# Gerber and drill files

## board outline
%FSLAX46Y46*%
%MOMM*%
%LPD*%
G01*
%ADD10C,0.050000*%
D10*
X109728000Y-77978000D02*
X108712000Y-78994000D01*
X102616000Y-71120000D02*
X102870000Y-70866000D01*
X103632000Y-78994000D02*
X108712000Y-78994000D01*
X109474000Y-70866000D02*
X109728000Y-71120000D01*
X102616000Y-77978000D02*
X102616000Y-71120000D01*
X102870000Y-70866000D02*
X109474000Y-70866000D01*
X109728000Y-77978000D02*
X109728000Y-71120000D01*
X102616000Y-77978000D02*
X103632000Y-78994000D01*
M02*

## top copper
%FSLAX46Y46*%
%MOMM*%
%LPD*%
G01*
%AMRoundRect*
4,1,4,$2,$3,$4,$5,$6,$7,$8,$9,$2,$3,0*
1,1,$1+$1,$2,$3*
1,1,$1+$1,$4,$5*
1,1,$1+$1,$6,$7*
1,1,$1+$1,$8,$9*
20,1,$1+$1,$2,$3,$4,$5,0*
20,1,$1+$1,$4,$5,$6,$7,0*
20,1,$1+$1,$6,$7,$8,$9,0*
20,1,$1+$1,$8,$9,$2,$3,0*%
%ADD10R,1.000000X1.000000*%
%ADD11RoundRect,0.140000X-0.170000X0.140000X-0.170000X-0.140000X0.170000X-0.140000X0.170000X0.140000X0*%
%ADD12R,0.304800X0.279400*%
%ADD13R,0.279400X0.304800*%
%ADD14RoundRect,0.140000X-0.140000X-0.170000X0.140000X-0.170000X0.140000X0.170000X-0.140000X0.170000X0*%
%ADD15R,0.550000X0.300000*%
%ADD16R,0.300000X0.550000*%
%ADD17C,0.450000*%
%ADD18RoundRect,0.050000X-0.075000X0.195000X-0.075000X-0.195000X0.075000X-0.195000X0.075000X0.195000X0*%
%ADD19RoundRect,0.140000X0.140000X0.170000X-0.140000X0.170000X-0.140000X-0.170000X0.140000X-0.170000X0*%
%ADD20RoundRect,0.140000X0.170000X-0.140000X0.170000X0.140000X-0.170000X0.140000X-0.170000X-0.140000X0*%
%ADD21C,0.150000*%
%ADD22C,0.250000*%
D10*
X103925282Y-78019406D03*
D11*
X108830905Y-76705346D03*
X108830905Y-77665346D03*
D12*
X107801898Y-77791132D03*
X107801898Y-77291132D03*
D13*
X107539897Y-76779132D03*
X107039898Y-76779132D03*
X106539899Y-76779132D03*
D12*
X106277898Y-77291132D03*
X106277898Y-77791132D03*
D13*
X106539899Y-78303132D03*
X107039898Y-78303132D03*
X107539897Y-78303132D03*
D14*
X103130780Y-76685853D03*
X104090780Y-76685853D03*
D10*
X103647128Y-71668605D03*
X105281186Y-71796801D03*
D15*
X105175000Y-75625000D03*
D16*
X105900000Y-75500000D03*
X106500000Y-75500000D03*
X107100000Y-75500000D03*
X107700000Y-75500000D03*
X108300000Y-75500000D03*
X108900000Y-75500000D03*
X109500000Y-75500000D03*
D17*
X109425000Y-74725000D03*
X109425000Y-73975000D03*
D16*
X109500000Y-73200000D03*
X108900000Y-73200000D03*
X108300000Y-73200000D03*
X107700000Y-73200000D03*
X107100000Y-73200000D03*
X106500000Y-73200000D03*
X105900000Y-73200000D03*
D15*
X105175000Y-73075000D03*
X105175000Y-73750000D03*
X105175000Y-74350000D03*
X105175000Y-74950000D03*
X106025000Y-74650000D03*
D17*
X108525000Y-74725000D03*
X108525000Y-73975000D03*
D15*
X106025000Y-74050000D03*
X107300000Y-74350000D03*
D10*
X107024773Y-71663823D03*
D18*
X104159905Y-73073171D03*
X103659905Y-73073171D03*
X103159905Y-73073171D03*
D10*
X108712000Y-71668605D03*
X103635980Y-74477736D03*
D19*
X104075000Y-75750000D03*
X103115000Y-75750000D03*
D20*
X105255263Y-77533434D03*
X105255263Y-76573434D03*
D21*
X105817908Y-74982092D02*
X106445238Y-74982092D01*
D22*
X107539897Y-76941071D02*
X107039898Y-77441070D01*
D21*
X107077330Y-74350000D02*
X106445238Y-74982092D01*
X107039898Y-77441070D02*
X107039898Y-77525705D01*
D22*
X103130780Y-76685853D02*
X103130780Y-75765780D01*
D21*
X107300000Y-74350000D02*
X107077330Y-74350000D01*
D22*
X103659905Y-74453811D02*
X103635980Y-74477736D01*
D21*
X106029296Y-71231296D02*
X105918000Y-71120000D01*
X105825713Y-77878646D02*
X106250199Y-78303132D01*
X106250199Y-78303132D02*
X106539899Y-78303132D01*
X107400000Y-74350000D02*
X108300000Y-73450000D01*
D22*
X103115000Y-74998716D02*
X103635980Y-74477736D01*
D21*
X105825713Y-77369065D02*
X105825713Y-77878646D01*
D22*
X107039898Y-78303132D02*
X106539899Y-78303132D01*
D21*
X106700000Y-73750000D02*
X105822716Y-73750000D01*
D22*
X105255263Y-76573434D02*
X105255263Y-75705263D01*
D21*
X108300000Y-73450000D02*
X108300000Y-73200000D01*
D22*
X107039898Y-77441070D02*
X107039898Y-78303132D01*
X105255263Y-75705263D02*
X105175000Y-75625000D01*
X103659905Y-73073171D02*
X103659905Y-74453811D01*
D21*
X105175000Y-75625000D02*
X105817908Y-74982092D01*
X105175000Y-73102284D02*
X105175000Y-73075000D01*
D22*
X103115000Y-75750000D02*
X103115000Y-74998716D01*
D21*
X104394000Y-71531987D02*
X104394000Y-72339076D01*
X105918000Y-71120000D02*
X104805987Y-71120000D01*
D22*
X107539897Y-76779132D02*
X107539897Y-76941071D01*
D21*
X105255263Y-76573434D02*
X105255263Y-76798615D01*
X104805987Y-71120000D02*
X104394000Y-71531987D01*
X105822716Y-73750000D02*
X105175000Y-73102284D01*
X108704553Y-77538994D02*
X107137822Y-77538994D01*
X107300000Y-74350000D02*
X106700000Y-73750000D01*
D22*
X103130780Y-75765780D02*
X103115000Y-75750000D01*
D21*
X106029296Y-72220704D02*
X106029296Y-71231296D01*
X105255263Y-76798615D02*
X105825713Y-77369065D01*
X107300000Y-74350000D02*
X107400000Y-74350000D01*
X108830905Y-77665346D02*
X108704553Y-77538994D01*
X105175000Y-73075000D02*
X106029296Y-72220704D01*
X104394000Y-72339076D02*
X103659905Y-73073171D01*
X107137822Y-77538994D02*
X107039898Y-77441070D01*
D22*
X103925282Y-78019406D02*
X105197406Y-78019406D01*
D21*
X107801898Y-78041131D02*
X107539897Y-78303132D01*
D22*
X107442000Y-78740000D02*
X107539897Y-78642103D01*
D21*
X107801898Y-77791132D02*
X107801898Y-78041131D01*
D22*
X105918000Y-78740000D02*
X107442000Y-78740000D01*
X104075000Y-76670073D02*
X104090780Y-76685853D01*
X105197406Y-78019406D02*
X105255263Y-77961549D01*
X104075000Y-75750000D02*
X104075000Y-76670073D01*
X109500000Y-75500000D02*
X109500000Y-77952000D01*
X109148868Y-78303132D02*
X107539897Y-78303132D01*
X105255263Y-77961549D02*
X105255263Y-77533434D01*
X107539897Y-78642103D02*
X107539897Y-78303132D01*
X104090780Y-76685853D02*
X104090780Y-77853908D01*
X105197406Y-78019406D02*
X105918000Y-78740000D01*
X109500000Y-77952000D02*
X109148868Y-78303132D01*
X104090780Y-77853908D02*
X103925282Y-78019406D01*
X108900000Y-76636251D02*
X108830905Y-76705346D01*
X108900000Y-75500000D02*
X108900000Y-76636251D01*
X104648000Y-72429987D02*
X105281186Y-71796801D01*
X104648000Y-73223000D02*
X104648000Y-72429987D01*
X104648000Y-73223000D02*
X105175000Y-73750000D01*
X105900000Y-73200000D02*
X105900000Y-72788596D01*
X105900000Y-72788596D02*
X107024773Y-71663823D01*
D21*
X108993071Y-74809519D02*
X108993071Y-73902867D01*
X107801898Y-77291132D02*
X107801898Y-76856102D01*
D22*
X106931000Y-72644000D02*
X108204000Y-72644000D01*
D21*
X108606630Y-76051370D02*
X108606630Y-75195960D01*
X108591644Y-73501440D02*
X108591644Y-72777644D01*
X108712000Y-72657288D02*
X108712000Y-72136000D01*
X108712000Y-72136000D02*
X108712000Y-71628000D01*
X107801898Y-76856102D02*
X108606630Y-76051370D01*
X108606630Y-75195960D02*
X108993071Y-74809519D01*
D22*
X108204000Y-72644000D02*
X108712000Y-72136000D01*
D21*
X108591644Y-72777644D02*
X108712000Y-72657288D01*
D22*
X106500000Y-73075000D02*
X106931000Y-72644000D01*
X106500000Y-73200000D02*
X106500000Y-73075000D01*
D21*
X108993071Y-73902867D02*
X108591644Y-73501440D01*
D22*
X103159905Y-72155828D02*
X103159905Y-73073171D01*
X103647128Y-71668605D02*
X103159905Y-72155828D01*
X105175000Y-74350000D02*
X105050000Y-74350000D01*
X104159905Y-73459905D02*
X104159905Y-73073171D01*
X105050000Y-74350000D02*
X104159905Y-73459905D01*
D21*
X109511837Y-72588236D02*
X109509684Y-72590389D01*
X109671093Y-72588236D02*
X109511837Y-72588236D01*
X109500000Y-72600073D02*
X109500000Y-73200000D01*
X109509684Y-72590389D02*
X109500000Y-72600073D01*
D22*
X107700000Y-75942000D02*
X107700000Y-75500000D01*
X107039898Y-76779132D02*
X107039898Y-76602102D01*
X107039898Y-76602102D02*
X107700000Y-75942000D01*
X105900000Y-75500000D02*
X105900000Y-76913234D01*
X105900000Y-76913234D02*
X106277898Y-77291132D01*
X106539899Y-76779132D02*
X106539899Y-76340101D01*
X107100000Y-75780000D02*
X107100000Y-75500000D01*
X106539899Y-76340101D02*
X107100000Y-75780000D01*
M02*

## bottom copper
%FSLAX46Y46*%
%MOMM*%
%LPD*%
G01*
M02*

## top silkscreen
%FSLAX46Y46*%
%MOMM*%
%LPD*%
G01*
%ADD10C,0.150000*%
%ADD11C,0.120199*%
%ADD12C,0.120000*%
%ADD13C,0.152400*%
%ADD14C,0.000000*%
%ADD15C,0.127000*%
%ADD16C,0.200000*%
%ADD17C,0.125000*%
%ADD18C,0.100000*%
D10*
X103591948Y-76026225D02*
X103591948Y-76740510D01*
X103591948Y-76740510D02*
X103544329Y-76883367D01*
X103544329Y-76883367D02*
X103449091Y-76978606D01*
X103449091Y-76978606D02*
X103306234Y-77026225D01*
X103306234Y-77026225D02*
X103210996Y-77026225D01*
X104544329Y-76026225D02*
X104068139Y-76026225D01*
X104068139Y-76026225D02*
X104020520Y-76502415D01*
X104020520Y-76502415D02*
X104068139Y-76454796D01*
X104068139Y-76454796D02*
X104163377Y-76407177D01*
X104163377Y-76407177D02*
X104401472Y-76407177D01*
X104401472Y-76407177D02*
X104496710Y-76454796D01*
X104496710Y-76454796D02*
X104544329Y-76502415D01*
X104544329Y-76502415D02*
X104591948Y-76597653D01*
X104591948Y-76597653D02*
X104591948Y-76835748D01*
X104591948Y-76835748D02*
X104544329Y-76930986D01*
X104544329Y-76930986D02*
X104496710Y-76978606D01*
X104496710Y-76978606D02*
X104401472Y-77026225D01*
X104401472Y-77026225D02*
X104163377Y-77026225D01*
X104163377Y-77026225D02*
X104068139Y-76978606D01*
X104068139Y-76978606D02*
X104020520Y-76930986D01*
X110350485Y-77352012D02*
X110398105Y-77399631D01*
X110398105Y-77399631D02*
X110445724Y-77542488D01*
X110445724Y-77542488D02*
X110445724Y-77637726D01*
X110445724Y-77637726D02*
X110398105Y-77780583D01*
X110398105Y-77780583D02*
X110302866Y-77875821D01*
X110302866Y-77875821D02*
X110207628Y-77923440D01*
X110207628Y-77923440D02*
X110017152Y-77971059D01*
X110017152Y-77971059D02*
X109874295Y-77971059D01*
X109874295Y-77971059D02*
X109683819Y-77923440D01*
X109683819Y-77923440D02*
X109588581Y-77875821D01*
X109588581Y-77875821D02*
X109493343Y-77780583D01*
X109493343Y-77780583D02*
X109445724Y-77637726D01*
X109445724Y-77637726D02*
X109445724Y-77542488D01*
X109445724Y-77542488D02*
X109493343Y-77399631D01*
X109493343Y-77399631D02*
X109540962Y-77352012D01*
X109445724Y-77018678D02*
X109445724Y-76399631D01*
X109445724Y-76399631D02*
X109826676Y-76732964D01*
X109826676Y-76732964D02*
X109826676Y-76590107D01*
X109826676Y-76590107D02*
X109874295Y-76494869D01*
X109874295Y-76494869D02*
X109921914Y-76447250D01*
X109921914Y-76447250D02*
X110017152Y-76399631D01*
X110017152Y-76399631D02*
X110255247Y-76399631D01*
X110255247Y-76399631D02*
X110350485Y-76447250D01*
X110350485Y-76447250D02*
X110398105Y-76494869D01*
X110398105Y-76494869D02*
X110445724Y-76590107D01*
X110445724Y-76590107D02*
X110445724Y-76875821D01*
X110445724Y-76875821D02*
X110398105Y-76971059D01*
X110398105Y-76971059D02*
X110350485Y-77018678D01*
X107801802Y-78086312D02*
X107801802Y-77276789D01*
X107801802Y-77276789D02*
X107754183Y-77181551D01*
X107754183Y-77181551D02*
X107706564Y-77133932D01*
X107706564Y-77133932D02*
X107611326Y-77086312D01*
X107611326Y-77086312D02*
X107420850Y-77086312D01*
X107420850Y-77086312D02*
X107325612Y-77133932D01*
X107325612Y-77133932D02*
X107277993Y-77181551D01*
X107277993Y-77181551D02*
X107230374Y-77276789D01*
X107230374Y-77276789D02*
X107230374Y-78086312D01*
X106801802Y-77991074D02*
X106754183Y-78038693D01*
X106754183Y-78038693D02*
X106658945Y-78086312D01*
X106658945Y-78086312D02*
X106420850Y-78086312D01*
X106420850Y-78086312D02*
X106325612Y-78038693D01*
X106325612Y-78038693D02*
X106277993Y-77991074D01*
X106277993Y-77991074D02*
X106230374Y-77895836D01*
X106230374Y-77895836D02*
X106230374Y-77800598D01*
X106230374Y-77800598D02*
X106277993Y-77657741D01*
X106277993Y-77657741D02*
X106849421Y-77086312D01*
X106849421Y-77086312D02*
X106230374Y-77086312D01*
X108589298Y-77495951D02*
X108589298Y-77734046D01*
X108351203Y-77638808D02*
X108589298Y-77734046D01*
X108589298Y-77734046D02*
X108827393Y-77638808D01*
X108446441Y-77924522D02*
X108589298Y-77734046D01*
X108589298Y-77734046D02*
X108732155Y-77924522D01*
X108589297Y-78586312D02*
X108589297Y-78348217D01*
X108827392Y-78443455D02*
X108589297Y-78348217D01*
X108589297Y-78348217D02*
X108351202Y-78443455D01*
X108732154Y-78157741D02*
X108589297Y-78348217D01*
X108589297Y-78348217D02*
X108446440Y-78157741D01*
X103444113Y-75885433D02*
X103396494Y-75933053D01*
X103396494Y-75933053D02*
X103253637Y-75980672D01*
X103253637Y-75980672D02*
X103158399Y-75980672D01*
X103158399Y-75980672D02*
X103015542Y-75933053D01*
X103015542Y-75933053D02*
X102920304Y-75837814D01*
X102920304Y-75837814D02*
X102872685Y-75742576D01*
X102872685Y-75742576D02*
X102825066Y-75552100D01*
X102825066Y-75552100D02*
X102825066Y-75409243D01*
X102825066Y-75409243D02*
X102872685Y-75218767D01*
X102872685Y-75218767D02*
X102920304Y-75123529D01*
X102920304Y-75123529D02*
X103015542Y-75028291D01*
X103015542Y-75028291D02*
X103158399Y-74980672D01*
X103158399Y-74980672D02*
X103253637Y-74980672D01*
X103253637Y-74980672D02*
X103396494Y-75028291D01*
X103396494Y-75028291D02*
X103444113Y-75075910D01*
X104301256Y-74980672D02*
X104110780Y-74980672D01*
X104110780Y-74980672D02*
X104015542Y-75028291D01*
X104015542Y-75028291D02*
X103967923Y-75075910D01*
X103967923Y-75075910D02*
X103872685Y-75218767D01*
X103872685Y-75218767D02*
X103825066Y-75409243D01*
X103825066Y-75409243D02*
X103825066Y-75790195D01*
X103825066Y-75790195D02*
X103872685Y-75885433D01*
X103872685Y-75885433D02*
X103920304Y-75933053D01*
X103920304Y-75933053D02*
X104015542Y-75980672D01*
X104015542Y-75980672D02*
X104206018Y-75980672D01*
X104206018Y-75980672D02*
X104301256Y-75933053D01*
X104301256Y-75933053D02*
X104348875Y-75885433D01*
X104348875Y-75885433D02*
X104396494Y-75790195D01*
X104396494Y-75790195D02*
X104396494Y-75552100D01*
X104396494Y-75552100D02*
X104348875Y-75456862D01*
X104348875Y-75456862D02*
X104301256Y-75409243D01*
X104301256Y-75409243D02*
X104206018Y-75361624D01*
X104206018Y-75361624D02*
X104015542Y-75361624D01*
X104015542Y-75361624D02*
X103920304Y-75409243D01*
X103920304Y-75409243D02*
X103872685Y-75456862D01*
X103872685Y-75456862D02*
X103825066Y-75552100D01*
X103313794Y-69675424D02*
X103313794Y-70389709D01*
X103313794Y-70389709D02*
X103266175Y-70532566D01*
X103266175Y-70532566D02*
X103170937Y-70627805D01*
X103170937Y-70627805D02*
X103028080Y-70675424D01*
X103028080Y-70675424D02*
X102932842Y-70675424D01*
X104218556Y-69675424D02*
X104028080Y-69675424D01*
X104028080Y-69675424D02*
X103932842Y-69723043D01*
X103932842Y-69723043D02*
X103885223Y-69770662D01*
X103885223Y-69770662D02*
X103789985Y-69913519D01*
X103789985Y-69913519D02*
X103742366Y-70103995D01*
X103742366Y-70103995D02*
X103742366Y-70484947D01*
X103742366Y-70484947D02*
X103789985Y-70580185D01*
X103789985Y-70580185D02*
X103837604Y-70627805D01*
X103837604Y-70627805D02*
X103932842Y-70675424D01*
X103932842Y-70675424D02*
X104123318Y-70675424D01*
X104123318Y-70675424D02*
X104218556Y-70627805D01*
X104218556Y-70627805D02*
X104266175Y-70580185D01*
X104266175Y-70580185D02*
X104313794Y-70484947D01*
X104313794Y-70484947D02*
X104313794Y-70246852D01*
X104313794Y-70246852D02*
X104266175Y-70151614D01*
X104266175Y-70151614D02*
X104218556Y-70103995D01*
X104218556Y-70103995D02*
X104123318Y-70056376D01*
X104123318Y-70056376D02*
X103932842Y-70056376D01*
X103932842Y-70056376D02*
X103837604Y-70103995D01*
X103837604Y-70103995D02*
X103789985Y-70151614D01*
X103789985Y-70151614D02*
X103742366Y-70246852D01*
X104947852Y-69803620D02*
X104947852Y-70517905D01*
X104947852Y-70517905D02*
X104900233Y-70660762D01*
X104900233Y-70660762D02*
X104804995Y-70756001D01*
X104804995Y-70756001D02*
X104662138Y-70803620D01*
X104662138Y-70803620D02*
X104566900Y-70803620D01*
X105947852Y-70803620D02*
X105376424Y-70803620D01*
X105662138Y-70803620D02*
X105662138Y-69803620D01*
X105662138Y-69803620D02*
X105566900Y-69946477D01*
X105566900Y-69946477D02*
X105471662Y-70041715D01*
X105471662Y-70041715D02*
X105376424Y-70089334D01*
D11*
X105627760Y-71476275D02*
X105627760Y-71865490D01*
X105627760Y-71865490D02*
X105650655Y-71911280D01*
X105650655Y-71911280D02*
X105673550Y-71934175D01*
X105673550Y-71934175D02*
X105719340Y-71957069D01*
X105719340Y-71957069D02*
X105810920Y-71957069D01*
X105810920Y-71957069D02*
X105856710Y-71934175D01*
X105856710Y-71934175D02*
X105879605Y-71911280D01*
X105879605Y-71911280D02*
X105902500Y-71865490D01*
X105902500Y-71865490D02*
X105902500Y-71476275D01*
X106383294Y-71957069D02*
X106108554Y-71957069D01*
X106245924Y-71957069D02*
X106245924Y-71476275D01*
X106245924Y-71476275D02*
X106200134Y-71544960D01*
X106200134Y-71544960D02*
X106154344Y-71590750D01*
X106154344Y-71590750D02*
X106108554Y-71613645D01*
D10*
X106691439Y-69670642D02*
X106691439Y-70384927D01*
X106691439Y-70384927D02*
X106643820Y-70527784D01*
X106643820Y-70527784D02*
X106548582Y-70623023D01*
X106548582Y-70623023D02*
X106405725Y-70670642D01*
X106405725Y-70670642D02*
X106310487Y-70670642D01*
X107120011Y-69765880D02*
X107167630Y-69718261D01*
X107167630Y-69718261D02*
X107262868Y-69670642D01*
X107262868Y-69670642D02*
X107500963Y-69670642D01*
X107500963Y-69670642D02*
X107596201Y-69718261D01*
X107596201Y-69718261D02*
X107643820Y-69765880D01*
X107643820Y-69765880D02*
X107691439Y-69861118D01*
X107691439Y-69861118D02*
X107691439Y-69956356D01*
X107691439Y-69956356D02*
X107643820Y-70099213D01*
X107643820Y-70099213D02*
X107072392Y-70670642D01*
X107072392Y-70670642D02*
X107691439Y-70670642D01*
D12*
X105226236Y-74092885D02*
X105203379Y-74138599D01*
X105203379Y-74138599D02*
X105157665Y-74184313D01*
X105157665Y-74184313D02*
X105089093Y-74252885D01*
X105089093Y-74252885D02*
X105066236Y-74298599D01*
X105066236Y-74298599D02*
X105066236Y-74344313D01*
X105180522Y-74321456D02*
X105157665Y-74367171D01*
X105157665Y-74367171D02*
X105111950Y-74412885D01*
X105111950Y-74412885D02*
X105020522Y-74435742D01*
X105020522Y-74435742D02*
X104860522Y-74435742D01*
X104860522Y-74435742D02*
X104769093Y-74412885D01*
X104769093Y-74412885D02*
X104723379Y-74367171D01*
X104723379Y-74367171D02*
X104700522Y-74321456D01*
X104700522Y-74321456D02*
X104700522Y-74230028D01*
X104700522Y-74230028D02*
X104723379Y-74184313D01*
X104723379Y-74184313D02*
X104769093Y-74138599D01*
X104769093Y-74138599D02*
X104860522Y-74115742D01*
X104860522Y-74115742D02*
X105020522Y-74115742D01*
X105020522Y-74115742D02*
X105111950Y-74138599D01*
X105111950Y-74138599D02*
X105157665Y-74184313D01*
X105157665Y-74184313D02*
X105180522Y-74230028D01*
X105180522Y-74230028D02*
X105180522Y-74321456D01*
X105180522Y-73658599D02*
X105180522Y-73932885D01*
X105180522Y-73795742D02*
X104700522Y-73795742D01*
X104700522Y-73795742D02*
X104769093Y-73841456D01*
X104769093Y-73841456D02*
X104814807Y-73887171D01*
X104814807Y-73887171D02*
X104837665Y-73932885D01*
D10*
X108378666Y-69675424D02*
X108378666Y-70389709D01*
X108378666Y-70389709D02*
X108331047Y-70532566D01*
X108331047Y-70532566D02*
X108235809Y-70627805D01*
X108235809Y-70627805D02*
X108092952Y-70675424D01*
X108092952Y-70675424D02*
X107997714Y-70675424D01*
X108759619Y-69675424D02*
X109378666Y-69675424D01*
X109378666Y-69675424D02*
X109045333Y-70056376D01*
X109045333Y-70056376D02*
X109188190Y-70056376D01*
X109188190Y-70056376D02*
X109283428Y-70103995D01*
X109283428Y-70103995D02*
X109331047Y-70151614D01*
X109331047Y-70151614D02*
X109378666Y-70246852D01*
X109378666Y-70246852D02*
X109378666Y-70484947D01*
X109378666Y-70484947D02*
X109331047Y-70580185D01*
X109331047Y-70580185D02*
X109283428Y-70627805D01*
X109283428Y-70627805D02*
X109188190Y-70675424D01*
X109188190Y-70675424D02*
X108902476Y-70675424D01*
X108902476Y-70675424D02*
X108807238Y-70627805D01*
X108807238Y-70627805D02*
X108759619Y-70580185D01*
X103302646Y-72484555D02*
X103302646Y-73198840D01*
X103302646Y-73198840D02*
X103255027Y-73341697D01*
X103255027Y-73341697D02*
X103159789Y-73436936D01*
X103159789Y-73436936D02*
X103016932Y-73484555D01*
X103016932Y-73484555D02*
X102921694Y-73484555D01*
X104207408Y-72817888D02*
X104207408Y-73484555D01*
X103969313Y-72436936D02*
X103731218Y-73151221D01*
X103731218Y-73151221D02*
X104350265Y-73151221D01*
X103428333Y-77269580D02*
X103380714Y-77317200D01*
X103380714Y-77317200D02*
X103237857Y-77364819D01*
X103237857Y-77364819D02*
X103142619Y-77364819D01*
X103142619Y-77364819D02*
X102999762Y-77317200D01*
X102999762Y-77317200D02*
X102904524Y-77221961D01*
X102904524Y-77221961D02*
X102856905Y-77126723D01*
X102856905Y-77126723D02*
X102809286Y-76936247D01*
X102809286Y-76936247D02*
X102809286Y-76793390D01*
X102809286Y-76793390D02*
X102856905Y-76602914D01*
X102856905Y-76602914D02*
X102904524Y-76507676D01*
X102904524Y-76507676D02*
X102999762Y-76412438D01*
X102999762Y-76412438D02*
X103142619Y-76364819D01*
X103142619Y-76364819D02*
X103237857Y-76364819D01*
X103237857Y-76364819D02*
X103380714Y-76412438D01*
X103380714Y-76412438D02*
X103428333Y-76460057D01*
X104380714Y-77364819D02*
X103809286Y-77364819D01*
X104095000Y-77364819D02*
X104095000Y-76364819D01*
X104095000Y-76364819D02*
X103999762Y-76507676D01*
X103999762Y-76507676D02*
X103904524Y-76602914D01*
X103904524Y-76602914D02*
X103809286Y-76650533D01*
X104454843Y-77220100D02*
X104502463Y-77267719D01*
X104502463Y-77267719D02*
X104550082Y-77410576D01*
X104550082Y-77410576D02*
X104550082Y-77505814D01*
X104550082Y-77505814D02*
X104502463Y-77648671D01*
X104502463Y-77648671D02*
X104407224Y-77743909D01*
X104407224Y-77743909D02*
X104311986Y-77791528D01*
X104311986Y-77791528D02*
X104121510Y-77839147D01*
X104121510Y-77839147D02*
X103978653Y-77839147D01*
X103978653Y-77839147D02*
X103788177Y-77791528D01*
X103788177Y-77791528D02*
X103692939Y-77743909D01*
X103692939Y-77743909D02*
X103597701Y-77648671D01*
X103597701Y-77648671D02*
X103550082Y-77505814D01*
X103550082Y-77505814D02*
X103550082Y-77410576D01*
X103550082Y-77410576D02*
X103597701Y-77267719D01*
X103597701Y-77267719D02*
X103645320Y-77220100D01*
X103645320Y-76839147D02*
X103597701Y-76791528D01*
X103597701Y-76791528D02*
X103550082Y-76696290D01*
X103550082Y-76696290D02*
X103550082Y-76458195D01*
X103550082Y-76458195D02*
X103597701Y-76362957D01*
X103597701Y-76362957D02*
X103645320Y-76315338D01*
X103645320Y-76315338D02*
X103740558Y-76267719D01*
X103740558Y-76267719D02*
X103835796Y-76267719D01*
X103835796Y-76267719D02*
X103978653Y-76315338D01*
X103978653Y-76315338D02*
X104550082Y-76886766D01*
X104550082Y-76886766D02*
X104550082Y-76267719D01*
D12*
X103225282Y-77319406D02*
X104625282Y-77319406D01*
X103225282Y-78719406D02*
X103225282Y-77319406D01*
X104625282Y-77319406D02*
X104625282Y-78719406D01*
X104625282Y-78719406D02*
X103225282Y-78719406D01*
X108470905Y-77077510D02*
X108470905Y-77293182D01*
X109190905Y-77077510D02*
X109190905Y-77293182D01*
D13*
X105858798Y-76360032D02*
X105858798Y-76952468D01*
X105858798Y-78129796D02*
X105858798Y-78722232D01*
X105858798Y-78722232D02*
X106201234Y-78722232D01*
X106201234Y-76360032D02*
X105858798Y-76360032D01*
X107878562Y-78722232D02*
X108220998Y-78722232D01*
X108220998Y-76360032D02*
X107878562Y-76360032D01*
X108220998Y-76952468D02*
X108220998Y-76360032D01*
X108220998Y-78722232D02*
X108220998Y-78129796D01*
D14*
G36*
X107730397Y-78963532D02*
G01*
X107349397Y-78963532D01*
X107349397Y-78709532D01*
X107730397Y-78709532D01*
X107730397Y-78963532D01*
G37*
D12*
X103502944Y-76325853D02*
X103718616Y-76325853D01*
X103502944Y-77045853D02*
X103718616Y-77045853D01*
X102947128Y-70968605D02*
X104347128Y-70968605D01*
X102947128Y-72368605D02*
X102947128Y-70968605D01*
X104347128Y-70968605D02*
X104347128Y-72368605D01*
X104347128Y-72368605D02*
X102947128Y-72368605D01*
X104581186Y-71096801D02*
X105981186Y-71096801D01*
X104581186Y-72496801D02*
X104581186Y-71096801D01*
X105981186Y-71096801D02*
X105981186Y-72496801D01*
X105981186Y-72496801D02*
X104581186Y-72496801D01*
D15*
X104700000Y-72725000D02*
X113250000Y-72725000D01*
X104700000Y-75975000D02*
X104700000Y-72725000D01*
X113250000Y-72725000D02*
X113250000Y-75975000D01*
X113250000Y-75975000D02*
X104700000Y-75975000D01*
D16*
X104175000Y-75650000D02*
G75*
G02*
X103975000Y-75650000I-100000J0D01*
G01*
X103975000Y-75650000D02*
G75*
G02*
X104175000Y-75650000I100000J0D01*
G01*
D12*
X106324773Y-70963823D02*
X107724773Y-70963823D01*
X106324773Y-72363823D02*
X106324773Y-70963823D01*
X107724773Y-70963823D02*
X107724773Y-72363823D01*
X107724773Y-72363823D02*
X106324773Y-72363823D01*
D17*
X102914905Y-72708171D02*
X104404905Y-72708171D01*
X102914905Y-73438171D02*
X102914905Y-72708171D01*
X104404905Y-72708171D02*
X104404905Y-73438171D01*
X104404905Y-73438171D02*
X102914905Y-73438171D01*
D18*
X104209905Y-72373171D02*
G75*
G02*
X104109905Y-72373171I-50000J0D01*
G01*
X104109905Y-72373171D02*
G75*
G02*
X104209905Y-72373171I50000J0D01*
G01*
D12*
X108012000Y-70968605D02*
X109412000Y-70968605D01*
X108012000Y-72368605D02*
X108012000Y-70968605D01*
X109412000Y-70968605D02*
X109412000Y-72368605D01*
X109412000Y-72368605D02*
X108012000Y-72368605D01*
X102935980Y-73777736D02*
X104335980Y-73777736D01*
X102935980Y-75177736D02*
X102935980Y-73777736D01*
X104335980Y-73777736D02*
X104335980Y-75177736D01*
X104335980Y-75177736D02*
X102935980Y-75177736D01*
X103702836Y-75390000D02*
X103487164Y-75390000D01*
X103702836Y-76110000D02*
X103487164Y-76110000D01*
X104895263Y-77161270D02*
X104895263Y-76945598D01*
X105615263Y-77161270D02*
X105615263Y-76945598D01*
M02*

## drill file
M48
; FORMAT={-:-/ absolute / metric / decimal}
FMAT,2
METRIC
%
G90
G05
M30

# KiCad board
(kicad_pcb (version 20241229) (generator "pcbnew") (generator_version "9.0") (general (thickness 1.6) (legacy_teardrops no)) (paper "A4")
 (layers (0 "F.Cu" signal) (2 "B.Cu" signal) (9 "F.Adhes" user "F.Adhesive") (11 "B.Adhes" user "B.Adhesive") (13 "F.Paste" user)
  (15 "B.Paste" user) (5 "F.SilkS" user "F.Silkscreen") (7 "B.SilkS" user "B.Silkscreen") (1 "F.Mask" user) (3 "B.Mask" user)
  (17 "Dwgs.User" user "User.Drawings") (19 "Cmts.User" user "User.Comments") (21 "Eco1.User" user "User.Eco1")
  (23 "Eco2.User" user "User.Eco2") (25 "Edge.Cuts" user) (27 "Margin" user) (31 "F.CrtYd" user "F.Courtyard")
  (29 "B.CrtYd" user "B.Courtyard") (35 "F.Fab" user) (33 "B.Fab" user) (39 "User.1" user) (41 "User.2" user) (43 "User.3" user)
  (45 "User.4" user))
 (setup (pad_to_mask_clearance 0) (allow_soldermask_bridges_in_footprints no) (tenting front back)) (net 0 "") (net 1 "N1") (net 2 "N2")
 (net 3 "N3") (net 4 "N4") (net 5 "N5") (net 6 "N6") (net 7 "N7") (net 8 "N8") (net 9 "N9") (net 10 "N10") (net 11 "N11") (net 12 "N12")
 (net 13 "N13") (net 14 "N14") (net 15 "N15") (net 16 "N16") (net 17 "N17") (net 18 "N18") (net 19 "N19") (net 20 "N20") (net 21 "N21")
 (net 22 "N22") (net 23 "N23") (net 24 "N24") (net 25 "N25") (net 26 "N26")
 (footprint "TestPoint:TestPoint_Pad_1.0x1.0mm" (layer "F.Cu") (at 103.925282 78.019406)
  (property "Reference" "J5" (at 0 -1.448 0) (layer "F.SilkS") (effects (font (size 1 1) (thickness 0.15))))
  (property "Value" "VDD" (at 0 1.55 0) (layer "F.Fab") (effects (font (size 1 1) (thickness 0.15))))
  (fp_line (start -0.7 -0.7) (end 0.7 -0.7) (stroke (width 0.12) (type solid)) (layer "F.SilkS"))
  (fp_line (start -0.7 0.7) (end -0.7 -0.7) (stroke (width 0.12) (type solid)) (layer "F.SilkS"))
  (fp_line (start 0.7 -0.7) (end 0.7 0.7) (stroke (width 0.12) (type solid)) (layer "F.SilkS"))
  (fp_line (start 0.7 0.7) (end -0.7 0.7) (stroke (width 0.12) (type solid)) (layer "F.SilkS"))
  (pad "1" smd rect (at 0 0) (size 1 1) (layers "F.Cu" "F.Mask") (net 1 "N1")))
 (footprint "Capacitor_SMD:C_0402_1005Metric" (layer "F.Cu") (at 108.830905 77.185346 -90)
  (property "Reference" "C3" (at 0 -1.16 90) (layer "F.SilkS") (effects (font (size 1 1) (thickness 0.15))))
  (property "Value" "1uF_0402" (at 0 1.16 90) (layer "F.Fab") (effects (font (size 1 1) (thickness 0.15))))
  (fp_line (start -0.107836 0.36) (end 0.107836 0.36) (stroke (width 0.12) (type solid)) (layer "F.SilkS"))
  (fp_line (start -0.107836 -0.36) (end 0.107836 -0.36) (stroke (width 0.12) (type solid)) (layer "F.SilkS"))
  (pad "1" smd roundrect (at -0.48 0 270) (size 0.56 0.62) (layers "F.Cu" "F.Mask" "F.Paste") (roundrect_rratio 0.25) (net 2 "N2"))
  (pad "2" smd roundrect (at 0.48 0 270) (size 0.56 0.62) (layers "F.Cu" "F.Mask" "F.Paste") (roundrect_rratio 0.25) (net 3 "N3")))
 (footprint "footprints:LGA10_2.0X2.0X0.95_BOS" (layer "F.Cu") (at 107.039898 77.541132 180)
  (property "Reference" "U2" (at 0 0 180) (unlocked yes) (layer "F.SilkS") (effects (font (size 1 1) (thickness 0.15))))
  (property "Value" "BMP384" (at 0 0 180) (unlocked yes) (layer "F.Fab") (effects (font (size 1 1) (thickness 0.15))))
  (fp_line (start 1.1811 1.1811) (end 1.1811 0.588664) (stroke (width 0.1524) (type solid)) (layer "F.SilkS"))
  (fp_line (start 1.1811 -0.588664) (end 1.1811 -1.1811) (stroke (width 0.1524) (type solid)) (layer "F.SilkS"))
  (fp_line (start 1.1811 -1.1811) (end 0.838664 -1.1811) (stroke (width 0.1524) (type solid)) (layer "F.SilkS"))
  (fp_line (start 0.838664 1.1811) (end 1.1811 1.1811) (stroke (width 0.1524) (type solid)) (layer "F.SilkS"))
  (fp_line (start -0.838664 -1.1811) (end -1.1811 -1.1811) (stroke (width 0.1524) (type solid)) (layer "F.SilkS"))
  (fp_line (start -1.1811 1.1811) (end -0.838664 1.1811) (stroke (width 0.1524) (type solid)) (layer "F.SilkS"))
  (fp_line (start -1.1811 0.588664) (end -1.1811 1.1811) (stroke (width 0.1524) (type solid)) (layer "F.SilkS"))
  (fp_line (start -1.1811 -1.1811) (end -1.1811 -0.588664) (stroke (width 0.1524) (type solid)) (layer "F.SilkS"))
  (fp_poly
   (pts (xy -0.690499 -1.1684) (xy -0.690499 -1.4224) (xy -0.309499 -1.4224) (xy -0.309499 -1.1684)) (stroke (width 0) (type solid))
   (fill yes) (layer "F.SilkS"))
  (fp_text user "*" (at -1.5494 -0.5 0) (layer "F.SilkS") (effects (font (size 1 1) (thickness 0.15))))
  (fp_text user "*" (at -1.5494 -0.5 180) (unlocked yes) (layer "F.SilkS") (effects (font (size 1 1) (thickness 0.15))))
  (pad "1" smd rect (at -0.762 -0.25 270) (size 0.2794 0.3048) (layers "F.Cu" "F.Mask" "F.Paste") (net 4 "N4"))
  (pad "2" smd rect (at -0.762 0.25 270) (size 0.2794 0.3048) (layers "F.Cu" "F.Mask" "F.Paste") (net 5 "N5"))
  (pad "3" smd rect (at -0.499999 0.762 180) (size 0.2794 0.3048) (layers "F.Cu" "F.Mask" "F.Paste") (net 3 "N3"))
  (pad "4" smd rect (at 0 0.762 180) (size 0.2794 0.3048) (layers "F.Cu" "F.Mask" "F.Paste") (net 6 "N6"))
  (pad "5" smd rect (at 0.499999 0.762 180) (size 0.2794 0.3048) (layers "F.Cu" "F.Mask" "F.Paste") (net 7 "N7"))
  (pad "6" smd rect (at 0.762 0.25 270) (size 0.2794 0.3048) (layers "F.Cu" "F.Mask" "F.Paste") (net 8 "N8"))
  (pad "7" smd rect (at 0.762 -0.25 270) (size 0.2794 0.3048) (layers "F.Cu" "F.Mask" "F.Paste") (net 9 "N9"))
  (pad "8" smd rect (at 0.499999 -0.762 180) (size 0.2794 0.3048) (layers "F.Cu" "F.Mask" "F.Paste") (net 3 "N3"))
  (pad "9" smd rect (at 0 -0.762 180) (size 0.2794 0.3048) (layers "F.Cu" "F.Mask" "F.Paste") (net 3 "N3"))
  (pad "10" smd rect (at -0.499999 -0.762 180) (size 0.2794 0.3048) (layers "F.Cu" "F.Mask" "F.Paste") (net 1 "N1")))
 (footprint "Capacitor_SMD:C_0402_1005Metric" (layer "F.Cu") (at 103.61078 76.685853)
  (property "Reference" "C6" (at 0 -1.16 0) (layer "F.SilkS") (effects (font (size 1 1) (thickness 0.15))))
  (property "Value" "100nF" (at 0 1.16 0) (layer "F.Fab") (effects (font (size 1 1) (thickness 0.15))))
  (fp_line (start -0.107836 -0.36) (end 0.107836 -0.36) (stroke (width 0.12) (type solid)) (layer "F.SilkS"))
  (fp_line (start -0.107836 0.36) (end 0.107836 0.36) (stroke (width 0.12) (type solid)) (layer "F.SilkS"))
  (pad "1" smd roundrect (at -0.48 0) (size 0.56 0.62) (layers "F.Cu" "F.Mask" "F.Paste") (roundrect_rratio 0.25) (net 3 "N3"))
  (pad "2" smd roundrect (at 0.48 0) (size 0.56 0.62) (layers "F.Cu" "F.Mask" "F.Paste") (roundrect_rratio 0.25) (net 1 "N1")))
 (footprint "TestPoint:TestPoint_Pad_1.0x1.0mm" (layer "F.Cu") (at 103.647128 71.668605)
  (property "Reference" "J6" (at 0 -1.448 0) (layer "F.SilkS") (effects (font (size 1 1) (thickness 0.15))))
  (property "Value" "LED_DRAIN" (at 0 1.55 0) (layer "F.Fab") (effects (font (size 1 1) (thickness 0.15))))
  (fp_line (start -0.7 -0.7) (end 0.7 -0.7) (stroke (width 0.12) (type solid)) (layer "F.SilkS"))
  (fp_line (start -0.7 0.7) (end -0.7 -0.7) (stroke (width 0.12) (type solid)) (layer "F.SilkS"))
  (fp_line (start 0.7 -0.7) (end 0.7 0.7) (stroke (width 0.12) (type solid)) (layer "F.SilkS"))
  (fp_line (start 0.7 0.7) (end -0.7 0.7) (stroke (width 0.12) (type solid)) (layer "F.SilkS"))
  (pad "1" smd rect (at 0 0) (size 1 1) (layers "F.Cu" "F.Mask") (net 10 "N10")))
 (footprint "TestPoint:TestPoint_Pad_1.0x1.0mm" (layer "F.Cu") (at 105.281186 71.796801)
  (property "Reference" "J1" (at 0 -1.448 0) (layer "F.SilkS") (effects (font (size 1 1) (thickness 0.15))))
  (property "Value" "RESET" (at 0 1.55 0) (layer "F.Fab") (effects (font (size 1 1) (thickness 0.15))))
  (fp_line (start -0.7 -0.7) (end 0.7 -0.7) (stroke (width 0.12) (type solid)) (layer "F.SilkS"))
  (fp_line (start -0.7 0.7) (end -0.7 -0.7) (stroke (width 0.12) (type solid)) (layer "F.SilkS"))
  (fp_line (start 0.7 -0.7) (end 0.7 0.7) (stroke (width 0.12) (type solid)) (layer "F.SilkS"))
  (fp_line (start 0.7 0.7) (end -0.7 0.7) (stroke (width 0.12) (type solid)) (layer "F.SilkS"))
  (pad "1" smd rect (at 0 0) (size 1 1) (layers "F.Cu" "F.Mask") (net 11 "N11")))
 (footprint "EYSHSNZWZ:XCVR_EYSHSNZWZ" (layer "F.Cu") (at 108.975 74.35)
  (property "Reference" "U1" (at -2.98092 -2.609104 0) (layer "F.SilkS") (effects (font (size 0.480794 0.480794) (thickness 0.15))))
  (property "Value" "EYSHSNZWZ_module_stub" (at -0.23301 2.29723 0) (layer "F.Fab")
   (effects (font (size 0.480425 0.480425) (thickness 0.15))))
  (fp_line (start -4.275 -1.625) (end 4.275 -1.625) (stroke (width 0.127) (type solid)) (layer "F.SilkS"))
  (fp_line (start -4.275 1.625) (end -4.275 -1.625) (stroke (width 0.127) (type solid)) (layer "F.SilkS"))
  (fp_line (start 4.275 -1.625) (end 4.275 1.625) (stroke (width 0.127) (type solid)) (layer "F.SilkS"))
  (fp_line (start 4.275 1.625) (end -4.275 1.625) (stroke (width 0.127) (type solid)) (layer "F.SilkS"))
  (fp_circle (center -4.9 1.3) (end -4.8 1.3) (stroke (width 0.2) (type solid)) (fill no) (layer "F.SilkS"))
  (pad "1" smd rect (at -3.8 1.275) (size 0.55 0.3) (layers "F.Cu" "F.Mask") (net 3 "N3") (solder_mask_margin 0.102))
  (pad "2" smd rect (at -3.075 1.15) (size 0.3 0.55) (layers "F.Cu" "F.Mask") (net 8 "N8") (solder_mask_margin 0.102))
  (pad "3" smd rect (at -2.475 1.15) (size 0.3 0.55) (layers "F.Cu" "F.Mask") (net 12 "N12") (solder_mask_margin 0.102))
  (pad "4" smd rect (at -1.875 1.15) (size 0.3 0.55) (layers "F.Cu" "F.Mask") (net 7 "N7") (solder_mask_margin 0.102))
  (pad "5" smd rect (at -1.275 1.15) (size 0.3 0.55) (layers "F.Cu" "F.Mask") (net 6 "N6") (solder_mask_margin 0.102))
  (pad "6" smd rect (at -0.675 1.15) (size 0.3 0.55) (layers "F.Cu" "F.Mask") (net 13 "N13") (solder_mask_margin 0.102))
  (pad "7" smd rect (at -0.075 1.15) (size 0.3 0.55) (layers "F.Cu" "F.Mask") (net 2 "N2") (solder_mask_margin 0.102))
  (pad "8" smd rect (at 0.525 1.15) (size 0.3 0.55) (layers "F.Cu" "F.Mask") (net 1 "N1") (solder_mask_margin 0.102))
  (pad "9" smd circle (at 0.45 0.375) (size 0.45 0.45) (layers "F.Cu" "F.Mask") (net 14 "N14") (solder_mask_margin 0.102))
  (pad "10" smd circle (at 0.45 -0.375) (size 0.45 0.45) (layers "F.Cu" "F.Mask") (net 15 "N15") (solder_mask_margin 0.102))
  (pad "11" smd rect (at 0.525 -1.15) (size 0.3 0.55) (layers "F.Cu" "F.Mask") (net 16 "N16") (solder_mask_margin 0.102))
  (pad "12" smd rect (at -0.075 -1.15) (size 0.3 0.55) (layers "F.Cu" "F.Mask") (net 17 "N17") (solder_mask_margin 0.102))
  (pad "13" smd rect (at -0.675 -1.15) (size 0.3 0.55) (layers "F.Cu" "F.Mask") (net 3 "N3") (solder_mask_margin 0.102))
  (pad "14" smd rect (at -1.275 -1.15) (size 0.3 0.55) (layers "F.Cu" "F.Mask") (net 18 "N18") (solder_mask_margin 0.102))
  (pad "15" smd rect (at -1.875 -1.15) (size 0.3 0.55) (layers "F.Cu" "F.Mask") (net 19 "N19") (solder_mask_margin 0.102))
  (pad "16" smd rect (at -2.475 -1.15) (size 0.3 0.55) (layers "F.Cu" "F.Mask") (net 5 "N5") (solder_mask_margin 0.102))
  (pad "17" smd rect (at -3.075 -1.15) (size 0.3 0.55) (layers "F.Cu" "F.Mask") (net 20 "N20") (solder_mask_margin 0.102))
  (pad "18" smd rect (at -3.8 -1.275) (size 0.55 0.3) (layers "F.Cu" "F.Mask") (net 3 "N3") (solder_mask_margin 0.102))
  (pad "19" smd rect (at -3.8 -0.6) (size 0.55 0.3) (layers "F.Cu" "F.Mask") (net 11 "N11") (solder_mask_margin 0.102))
  (pad "20" smd rect (at -3.8 0) (size 0.55 0.3) (layers "F.Cu" "F.Mask") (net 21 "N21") (solder_mask_margin 0.102))
  (pad "21" smd rect (at -3.8 0.6) (size 0.55 0.3) (layers "F.Cu" "F.Mask") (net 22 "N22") (solder_mask_margin 0.102))
  (pad "22" smd rect (at -2.95 0.3) (size 0.55 0.3) (layers "F.Cu" "F.Mask") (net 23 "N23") (solder_mask_margin 0.102))
  (pad "23" smd circle (at -0.45 0.375) (size 0.45 0.45) (layers "F.Cu" "F.Mask") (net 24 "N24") (solder_mask_margin 0.102))
  (pad "24" smd circle (at -0.45 -0.375) (size 0.45 0.45) (layers "F.Cu" "F.Mask") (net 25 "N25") (solder_mask_margin 0.102))
  (pad "25" smd rect (at -2.95 -0.3) (size 0.55 0.3) (layers "F.Cu" "F.Mask") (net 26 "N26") (solder_mask_margin 0.102))
  (pad "26" smd rect (at -1.675 0) (size 0.55 0.3) (layers "F.Cu" "F.Mask") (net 3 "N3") (solder_mask_margin 0.102)))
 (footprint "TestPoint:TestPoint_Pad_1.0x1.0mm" (layer "F.Cu") (at 107.024773 71.663823)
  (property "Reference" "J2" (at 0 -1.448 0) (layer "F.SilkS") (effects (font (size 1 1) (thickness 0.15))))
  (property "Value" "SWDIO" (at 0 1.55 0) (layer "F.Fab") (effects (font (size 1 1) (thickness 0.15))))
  (fp_line (start -0.7 -0.7) (end 0.7 -0.7) (stroke (width 0.12) (type solid)) (layer "F.SilkS"))
  (fp_line (start -0.7 0.7) (end -0.7 -0.7) (stroke (width 0.12) (type solid)) (layer "F.SilkS"))
  (fp_line (start 0.7 -0.7) (end 0.7 0.7) (stroke (width 0.12) (type solid)) (layer "F.SilkS"))
  (fp_line (start 0.7 0.7) (end -0.7 0.7) (stroke (width 0.12) (type solid)) (layer "F.SilkS"))
  (pad "1" smd rect (at 0 0) (size 1 1) (layers "F.Cu" "F.Mask") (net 20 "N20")))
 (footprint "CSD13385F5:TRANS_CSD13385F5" (layer "F.Cu") (at 103.659905 73.073171 -90)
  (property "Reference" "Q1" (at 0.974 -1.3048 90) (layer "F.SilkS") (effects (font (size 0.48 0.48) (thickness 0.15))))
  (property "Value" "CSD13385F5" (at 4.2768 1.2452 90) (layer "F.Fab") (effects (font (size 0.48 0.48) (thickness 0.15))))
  (fp_line (start -0.365 0.745) (end -0.365 -0.745) (stroke (width 0.125) (type solid)) (layer "F.SilkS"))
  (fp_line (start 0.365 0.745) (end -0.365 0.745) (stroke (width 0.125) (type solid)) (layer "F.SilkS"))
  (fp_line (start -0.365 -0.745) (end 0.365 -0.745) (stroke (width 0.125) (type solid)) (layer "F.SilkS"))
  (fp_line (start 0.365 -0.745) (end 0.365 0.745) (stroke (width 0.125) (type solid)) (layer "F.SilkS"))
  (fp_circle (center -0.7 -0.5) (end -0.65 -0.5) (stroke (width 0.1) (type solid)) (fill no) (layer "F.SilkS"))
  (pad "1" smd roundrect (at 0 -0.5 270) (size 0.49 0.25) (layers "F.Cu") (roundrect_rratio 0.2) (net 21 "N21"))
  (pad "2" smd roundrect (at 0 0 270) (size 0.49 0.25) (layers "F.Cu") (roundrect_rratio 0.2) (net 3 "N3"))
  (pad "3" smd roundrect (at 0 0.5 270) (size 0.49 0.25) (layers "F.Cu") (roundrect_rratio 0.2) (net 10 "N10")))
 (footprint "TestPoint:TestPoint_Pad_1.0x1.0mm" (layer "F.Cu") (at 108.712 71.668605)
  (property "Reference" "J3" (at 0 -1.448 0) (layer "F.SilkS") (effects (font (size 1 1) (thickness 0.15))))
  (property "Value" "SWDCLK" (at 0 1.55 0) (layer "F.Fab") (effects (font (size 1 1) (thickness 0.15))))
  (fp_line (start -0.7 -0.7) (end 0.7 -0.7) (stroke (width 0.12) (type solid)) (layer "F.SilkS"))
  (fp_line (start -0.7 0.7) (end -0.7 -0.7) (stroke (width 0.12) (type solid)) (layer "F.SilkS"))
  (fp_line (start 0.7 -0.7) (end 0.7 0.7) (stroke (width 0.12) (type solid)) (layer "F.SilkS"))
  (fp_line (start 0.7 0.7) (end -0.7 0.7) (stroke (width 0.12) (type solid)) (layer "F.SilkS"))
  (pad "1" smd rect (at 0 0) (size 1 1) (layers "F.Cu" "F.Mask") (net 5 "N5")))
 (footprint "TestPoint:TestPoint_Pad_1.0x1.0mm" (layer "F.Cu") (at 103.63598 74.477736)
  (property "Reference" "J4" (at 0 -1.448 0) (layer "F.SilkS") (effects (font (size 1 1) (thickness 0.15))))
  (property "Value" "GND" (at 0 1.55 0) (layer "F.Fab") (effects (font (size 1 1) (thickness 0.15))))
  (fp_line (start -0.7 -0.7) (end 0.7 -0.7) (stroke (width 0.12) (type solid)) (layer "F.SilkS"))
  (fp_line (start -0.7 0.7) (end -0.7 -0.7) (stroke (width 0.12) (type solid)) (layer "F.SilkS"))
  (fp_line (start 0.7 -0.7) (end 0.7 0.7) (stroke (width 0.12) (type solid)) (layer "F.SilkS"))
  (fp_line (start 0.7 0.7) (end -0.7 0.7) (stroke (width 0.12) (type solid)) (layer "F.SilkS"))
  (pad "1" smd rect (at 0 0) (size 1 1) (layers "F.Cu" "F.Mask") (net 3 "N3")))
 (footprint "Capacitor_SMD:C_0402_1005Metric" (layer "F.Cu") (at 103.595 75.75 180)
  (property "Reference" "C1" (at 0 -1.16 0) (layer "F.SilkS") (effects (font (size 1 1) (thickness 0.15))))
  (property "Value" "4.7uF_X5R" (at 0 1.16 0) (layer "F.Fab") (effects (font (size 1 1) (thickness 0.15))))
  (fp_line (start -0.107836 0.36) (end 0.107836 0.36) (stroke (width 0.12) (type solid)) (layer "F.SilkS"))
  (fp_line (start -0.107836 -0.36) (end 0.107836 -0.36) (stroke (width 0.12) (type solid)) (layer "F.SilkS"))
  (pad "1" smd roundrect (at -0.48 0 180) (size 0.56 0.62) (layers "F.Cu" "F.Mask" "F.Paste") (roundrect_rratio 0.25) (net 1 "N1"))
  (pad "2" smd roundrect (at 0.48 0 180) (size 0.56 0.62) (layers "F.Cu" "F.Mask" "F.Paste") (roundrect_rratio 0.25) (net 3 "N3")))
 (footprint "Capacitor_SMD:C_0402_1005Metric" (layer "F.Cu") (at 105.255263 77.053434 90)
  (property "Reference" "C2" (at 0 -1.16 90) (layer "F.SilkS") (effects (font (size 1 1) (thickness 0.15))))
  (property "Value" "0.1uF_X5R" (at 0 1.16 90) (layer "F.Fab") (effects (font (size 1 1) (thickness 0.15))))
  (fp_line (start -0.107836 -0.36) (end 0.107836 -0.36) (stroke (width 0.12) (type solid)) (layer "F.SilkS"))
  (fp_line (start -0.107836 0.36) (end 0.107836 0.36) (stroke (width 0.12) (type solid)) (layer "F.SilkS"))
  (pad "1" smd roundrect (at -0.48 0 90) (size 0.56 0.62) (layers "F.Cu" "F.Mask" "F.Paste") (roundrect_rratio 0.25) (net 1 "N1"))
  (pad "2" smd roundrect (at 0.48 0 90) (size 0.56 0.62) (layers "F.Cu" "F.Mask" "F.Paste") (roundrect_rratio 0.25) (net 3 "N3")))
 (gr_line (start 109.728 77.978) (end 108.712 78.994) (stroke (width 0.05) (type default)) (layer "Edge.Cuts"))
 (gr_line (start 102.616 71.12) (end 102.87 70.866) (stroke (width 0.05) (type default)) (layer "Edge.Cuts"))
 (gr_line (start 103.632 78.994) (end 108.712 78.994) (stroke (width 0.05) (type default)) (layer "Edge.Cuts"))
 (gr_line (start 109.474 70.866) (end 109.728 71.12) (stroke (width 0.05) (type default)) (layer "Edge.Cuts"))
 (gr_line (start 102.616 77.978) (end 102.616 71.12) (stroke (width 0.05) (type default)) (layer "Edge.Cuts"))
 (gr_line (start 102.87 70.866) (end 109.474 70.866) (stroke (width 0.05) (type default)) (layer "Edge.Cuts"))
 (gr_line (start 109.728 77.978) (end 109.728 71.12) (stroke (width 0.05) (type default)) (layer "Edge.Cuts"))
 (gr_line (start 102.616 77.978) (end 103.632 78.994) (stroke (width 0.05) (type default)) (layer "Edge.Cuts"))
 (segment (start 105.817908 74.982092) (end 106.445238 74.982092) (width 0.15) (layer "F.Cu") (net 3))
 (segment (start 107.539897 76.941071) (end 107.039898 77.44107) (width 0.25) (layer "F.Cu") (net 3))
 (segment (start 107.07733 74.35) (end 106.445238 74.982092) (width 0.15) (layer "F.Cu") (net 3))
 (segment (start 107.039898 77.44107) (end 107.039898 77.525705) (width 0.15) (layer "F.Cu") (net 3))
 (segment (start 103.13078 76.685853) (end 103.13078 75.76578) (width 0.25) (layer "F.Cu") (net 3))
 (segment (start 107.3 74.35) (end 107.07733 74.35) (width 0.15) (layer "F.Cu") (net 3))
 (segment (start 103.659905 74.453811) (end 103.63598 74.477736) (width 0.25) (layer "F.Cu") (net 3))
 (segment (start 106.029296 71.231296) (end 105.918 71.12) (width 0.15) (layer "F.Cu") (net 3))
 (segment (start 105.825713 77.878646) (end 106.250199 78.303132) (width 0.15) (layer "F.Cu") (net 3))
 (segment (start 106.250199 78.303132) (end 106.539899 78.303132) (width 0.15) (layer "F.Cu") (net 3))
 (segment (start 107.4 74.35) (end 108.3 73.45) (width 0.15) (layer "F.Cu") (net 3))
 (segment (start 103.115 74.998716) (end 103.63598 74.477736) (width 0.25) (layer "F.Cu") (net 3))
 (segment (start 105.825713 77.369065) (end 105.825713 77.878646) (width 0.15) (layer "F.Cu") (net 3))
 (segment (start 107.039898 78.303132) (end 106.539899 78.303132) (width 0.25) (layer "F.Cu") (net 3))
 (segment (start 106.7 73.75) (end 105.822716 73.75) (width 0.15) (layer "F.Cu") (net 3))
 (segment (start 105.255263 76.573434) (end 105.255263 75.705263) (width 0.25) (layer "F.Cu") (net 3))
 (segment (start 108.3 73.45) (end 108.3 73.2) (width 0.15) (layer "F.Cu") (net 3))
 (segment (start 107.039898 77.44107) (end 107.039898 78.303132) (width 0.25) (layer "F.Cu") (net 3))
 (segment (start 105.255263 75.705263) (end 105.175 75.625) (width 0.25) (layer "F.Cu") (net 3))
 (segment (start 103.659905 73.073171) (end 103.659905 74.453811) (width 0.25) (layer "F.Cu") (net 3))
 (segment (start 105.175 75.625) (end 105.817908 74.982092) (width 0.15) (layer "F.Cu") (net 3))
 (segment (start 105.175 73.102284) (end 105.175 73.075) (width 0.15) (layer "F.Cu") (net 3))
 (segment (start 103.115 75.75) (end 103.115 74.998716) (width 0.25) (layer "F.Cu") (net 3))
 (segment (start 104.394 71.531987) (end 104.394 72.339076) (width 0.15) (layer "F.Cu") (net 3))
 (segment (start 105.918 71.12) (end 104.805987 71.12) (width 0.15) (layer "F.Cu") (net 3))
 (segment (start 107.539897 76.779132) (end 107.539897 76.941071) (width 0.25) (layer "F.Cu") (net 3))
 (segment (start 105.255263 76.573434) (end 105.255263 76.798615) (width 0.15) (layer "F.Cu") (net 3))
 (segment (start 104.805987 71.12) (end 104.394 71.531987) (width 0.15) (layer "F.Cu") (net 3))
 (segment (start 105.822716 73.75) (end 105.175 73.102284) (width 0.15) (layer "F.Cu") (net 3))
 (segment (start 108.704553 77.538994) (end 107.137822 77.538994) (width 0.15) (layer "F.Cu") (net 3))
 (segment (start 107.3 74.35) (end 106.7 73.75) (width 0.15) (layer "F.Cu") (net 3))
 (segment (start 103.13078 75.76578) (end 103.115 75.75) (width 0.25) (layer "F.Cu") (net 3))
 (segment (start 106.029296 72.220704) (end 106.029296 71.231296) (width 0.15) (layer "F.Cu") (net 3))
 (segment (start 105.255263 76.798615) (end 105.825713 77.369065) (width 0.15) (layer "F.Cu") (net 3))
 (segment (start 107.3 74.35) (end 107.4 74.35) (width 0.15) (layer "F.Cu") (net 3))
 (segment (start 108.830905 77.665346) (end 108.704553 77.538994) (width 0.15) (layer "F.Cu") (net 3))
 (segment (start 105.175 73.075) (end 106.029296 72.220704) (width 0.15) (layer "F.Cu") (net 3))
 (segment (start 104.394 72.339076) (end 103.659905 73.073171) (width 0.15) (layer "F.Cu") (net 3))
 (segment (start 107.137822 77.538994) (end 107.039898 77.44107) (width 0.15) (layer "F.Cu") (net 3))
 (segment (start 103.925282 78.019406) (end 105.197406 78.019406) (width 0.25) (layer "F.Cu") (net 1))
 (segment (start 107.801898 78.041131) (end 107.539897 78.303132) (width 0.15) (layer "F.Cu") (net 1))
 (segment (start 107.442 78.74) (end 107.539897 78.642103) (width 0.25) (layer "F.Cu") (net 1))
 (segment (start 107.801898 77.791132) (end 107.801898 78.041131) (width 0.15) (layer "F.Cu") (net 1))
 (segment (start 105.918 78.74) (end 107.442 78.74) (width 0.25) (layer "F.Cu") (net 1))
 (segment (start 104.075 76.670073) (end 104.09078 76.685853) (width 0.25) (layer "F.Cu") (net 1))
 (segment (start 105.197406 78.019406) (end 105.255263 77.961549) (width 0.25) (layer "F.Cu") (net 1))
 (segment (start 104.075 75.75) (end 104.075 76.670073) (width 0.25) (layer "F.Cu") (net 1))
 (segment (start 109.5 75.5) (end 109.5 77.952) (width 0.25) (layer "F.Cu") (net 1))
 (segment (start 109.148868 78.303132) (end 107.539897 78.303132) (width 0.25) (layer "F.Cu") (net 1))
 (segment (start 105.255263 77.961549) (end 105.255263 77.533434) (width 0.25) (layer "F.Cu") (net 1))
 (segment (start 107.539897 78.642103) (end 107.539897 78.303132) (width 0.25) (layer "F.Cu") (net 1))
 (segment (start 104.09078 76.685853) (end 104.09078 77.853908) (width 0.25) (layer "F.Cu") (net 1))
 (segment (start 105.197406 78.019406) (end 105.918 78.74) (width 0.25) (layer "F.Cu") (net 1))
 (segment (start 109.5 77.952) (end 109.148868 78.303132) (width 0.25) (layer "F.Cu") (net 1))
 (segment (start 104.09078 77.853908) (end 103.925282 78.019406) (width 0.25) (layer "F.Cu") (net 1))
 (segment (start 108.9 76.636251) (end 108.830905 76.705346) (width 0.25) (layer "F.Cu") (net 2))
 (segment (start 108.9 75.5) (end 108.9 76.636251) (width 0.25) (layer "F.Cu") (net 2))
 (segment (start 104.648 72.429987) (end 105.281186 71.796801) (width 0.25) (layer "F.Cu") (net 11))
 (segment (start 104.648 73.223) (end 104.648 72.429987) (width 0.25) (layer "F.Cu") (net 11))
 (segment (start 104.648 73.223) (end 105.175 73.75) (width 0.25) (layer "F.Cu") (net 11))
 (segment (start 105.9 73.2) (end 105.9 72.788596) (width 0.25) (layer "F.Cu") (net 20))
 (segment (start 105.9 72.788596) (end 107.024773 71.663823) (width 0.25) (layer "F.Cu") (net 20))
 (segment (start 108.993071 74.809519) (end 108.993071 73.902867) (width 0.15) (layer "F.Cu") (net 5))
 (segment (start 107.801898 77.291132) (end 107.801898 76.856102) (width 0.15) (layer "F.Cu") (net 5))
 (segment (start 106.931 72.644) (end 108.204 72.644) (width 0.25) (layer "F.Cu") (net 5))
 (segment (start 108.60663 76.05137) (end 108.60663 75.19596) (width 0.15) (layer "F.Cu") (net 5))
 (segment (start 108.591644 73.50144) (end 108.591644 72.777644) (width 0.15) (layer "F.Cu") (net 5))
 (segment (start 108.712 72.657288) (end 108.712 72.136) (width 0.15) (layer "F.Cu") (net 5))
 (segment (start 108.712 72.136) (end 108.712 71.628) (width 0.15) (layer "F.Cu") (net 5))
 (segment (start 107.801898 76.856102) (end 108.60663 76.05137) (width 0.15) (layer "F.Cu") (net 5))
 (segment (start 108.60663 75.19596) (end 108.993071 74.809519) (width 0.15) (layer "F.Cu") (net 5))
 (segment (start 108.204 72.644) (end 108.712 72.136) (width 0.25) (layer "F.Cu") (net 5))
 (segment (start 108.591644 72.777644) (end 108.712 72.657288) (width 0.15) (layer "F.Cu") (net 5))
 (segment (start 106.5 73.075) (end 106.931 72.644) (width 0.25) (layer "F.Cu") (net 5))
 (segment (start 106.5 73.2) (end 106.5 73.075) (width 0.25) (layer "F.Cu") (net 5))
 (segment (start 108.993071 73.902867) (end 108.591644 73.50144) (width 0.15) (layer "F.Cu") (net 5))
 (segment (start 103.159905 72.155828) (end 103.159905 73.073171) (width 0.25) (layer "F.Cu") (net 10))
 (segment (start 103.647128 71.668605) (end 103.159905 72.155828) (width 0.25) (layer "F.Cu") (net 10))
 (segment (start 105.175 74.35) (end 105.05 74.35) (width 0.25) (layer "F.Cu") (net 21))
 (segment (start 104.159905 73.459905) (end 104.159905 73.073171) (width 0.25) (layer "F.Cu") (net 21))
 (segment (start 105.05 74.35) (end 104.159905 73.459905) (width 0.25) (layer "F.Cu") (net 21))
 (segment (start 109.511837 72.588236) (end 109.509684 72.590389) (width 0.15) (layer "F.Cu") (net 16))
 (segment (start 109.671093 72.588236) (end 109.511837 72.588236) (width 0.15) (layer "F.Cu") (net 16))
 (segment (start 109.5 72.600073) (end 109.5 73.2) (width 0.15) (layer "F.Cu") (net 16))
 (segment (start 109.509684 72.590389) (end 109.5 72.600073) (width 0.15) (layer "F.Cu") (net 16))
 (segment (start 107.7 75.942) (end 107.7 75.5) (width 0.25) (layer "F.Cu") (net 6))
 (segment (start 107.039898 76.779132) (end 107.039898 76.602102) (width 0.25) (layer "F.Cu") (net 6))
 (segment (start 107.039898 76.602102) (end 107.7 75.942) (width 0.25) (layer "F.Cu") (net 6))
 (segment (start 105.9 75.5) (end 105.9 76.913234) (width 0.25) (layer "F.Cu") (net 8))
 (segment (start 105.9 76.913234) (end 106.277898 77.291132) (width 0.25) (layer "F.Cu") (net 8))
 (segment (start 106.539899 76.779132) (end 106.539899 76.340101) (width 0.25) (layer "F.Cu") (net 7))
 (segment (start 107.1 75.78) (end 107.1 75.5) (width 0.25) (layer "F.Cu") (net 7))
 (segment (start 106.539899 76.340101) (end 107.1 75.78) (width 0.25) (layer "F.Cu") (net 7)))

